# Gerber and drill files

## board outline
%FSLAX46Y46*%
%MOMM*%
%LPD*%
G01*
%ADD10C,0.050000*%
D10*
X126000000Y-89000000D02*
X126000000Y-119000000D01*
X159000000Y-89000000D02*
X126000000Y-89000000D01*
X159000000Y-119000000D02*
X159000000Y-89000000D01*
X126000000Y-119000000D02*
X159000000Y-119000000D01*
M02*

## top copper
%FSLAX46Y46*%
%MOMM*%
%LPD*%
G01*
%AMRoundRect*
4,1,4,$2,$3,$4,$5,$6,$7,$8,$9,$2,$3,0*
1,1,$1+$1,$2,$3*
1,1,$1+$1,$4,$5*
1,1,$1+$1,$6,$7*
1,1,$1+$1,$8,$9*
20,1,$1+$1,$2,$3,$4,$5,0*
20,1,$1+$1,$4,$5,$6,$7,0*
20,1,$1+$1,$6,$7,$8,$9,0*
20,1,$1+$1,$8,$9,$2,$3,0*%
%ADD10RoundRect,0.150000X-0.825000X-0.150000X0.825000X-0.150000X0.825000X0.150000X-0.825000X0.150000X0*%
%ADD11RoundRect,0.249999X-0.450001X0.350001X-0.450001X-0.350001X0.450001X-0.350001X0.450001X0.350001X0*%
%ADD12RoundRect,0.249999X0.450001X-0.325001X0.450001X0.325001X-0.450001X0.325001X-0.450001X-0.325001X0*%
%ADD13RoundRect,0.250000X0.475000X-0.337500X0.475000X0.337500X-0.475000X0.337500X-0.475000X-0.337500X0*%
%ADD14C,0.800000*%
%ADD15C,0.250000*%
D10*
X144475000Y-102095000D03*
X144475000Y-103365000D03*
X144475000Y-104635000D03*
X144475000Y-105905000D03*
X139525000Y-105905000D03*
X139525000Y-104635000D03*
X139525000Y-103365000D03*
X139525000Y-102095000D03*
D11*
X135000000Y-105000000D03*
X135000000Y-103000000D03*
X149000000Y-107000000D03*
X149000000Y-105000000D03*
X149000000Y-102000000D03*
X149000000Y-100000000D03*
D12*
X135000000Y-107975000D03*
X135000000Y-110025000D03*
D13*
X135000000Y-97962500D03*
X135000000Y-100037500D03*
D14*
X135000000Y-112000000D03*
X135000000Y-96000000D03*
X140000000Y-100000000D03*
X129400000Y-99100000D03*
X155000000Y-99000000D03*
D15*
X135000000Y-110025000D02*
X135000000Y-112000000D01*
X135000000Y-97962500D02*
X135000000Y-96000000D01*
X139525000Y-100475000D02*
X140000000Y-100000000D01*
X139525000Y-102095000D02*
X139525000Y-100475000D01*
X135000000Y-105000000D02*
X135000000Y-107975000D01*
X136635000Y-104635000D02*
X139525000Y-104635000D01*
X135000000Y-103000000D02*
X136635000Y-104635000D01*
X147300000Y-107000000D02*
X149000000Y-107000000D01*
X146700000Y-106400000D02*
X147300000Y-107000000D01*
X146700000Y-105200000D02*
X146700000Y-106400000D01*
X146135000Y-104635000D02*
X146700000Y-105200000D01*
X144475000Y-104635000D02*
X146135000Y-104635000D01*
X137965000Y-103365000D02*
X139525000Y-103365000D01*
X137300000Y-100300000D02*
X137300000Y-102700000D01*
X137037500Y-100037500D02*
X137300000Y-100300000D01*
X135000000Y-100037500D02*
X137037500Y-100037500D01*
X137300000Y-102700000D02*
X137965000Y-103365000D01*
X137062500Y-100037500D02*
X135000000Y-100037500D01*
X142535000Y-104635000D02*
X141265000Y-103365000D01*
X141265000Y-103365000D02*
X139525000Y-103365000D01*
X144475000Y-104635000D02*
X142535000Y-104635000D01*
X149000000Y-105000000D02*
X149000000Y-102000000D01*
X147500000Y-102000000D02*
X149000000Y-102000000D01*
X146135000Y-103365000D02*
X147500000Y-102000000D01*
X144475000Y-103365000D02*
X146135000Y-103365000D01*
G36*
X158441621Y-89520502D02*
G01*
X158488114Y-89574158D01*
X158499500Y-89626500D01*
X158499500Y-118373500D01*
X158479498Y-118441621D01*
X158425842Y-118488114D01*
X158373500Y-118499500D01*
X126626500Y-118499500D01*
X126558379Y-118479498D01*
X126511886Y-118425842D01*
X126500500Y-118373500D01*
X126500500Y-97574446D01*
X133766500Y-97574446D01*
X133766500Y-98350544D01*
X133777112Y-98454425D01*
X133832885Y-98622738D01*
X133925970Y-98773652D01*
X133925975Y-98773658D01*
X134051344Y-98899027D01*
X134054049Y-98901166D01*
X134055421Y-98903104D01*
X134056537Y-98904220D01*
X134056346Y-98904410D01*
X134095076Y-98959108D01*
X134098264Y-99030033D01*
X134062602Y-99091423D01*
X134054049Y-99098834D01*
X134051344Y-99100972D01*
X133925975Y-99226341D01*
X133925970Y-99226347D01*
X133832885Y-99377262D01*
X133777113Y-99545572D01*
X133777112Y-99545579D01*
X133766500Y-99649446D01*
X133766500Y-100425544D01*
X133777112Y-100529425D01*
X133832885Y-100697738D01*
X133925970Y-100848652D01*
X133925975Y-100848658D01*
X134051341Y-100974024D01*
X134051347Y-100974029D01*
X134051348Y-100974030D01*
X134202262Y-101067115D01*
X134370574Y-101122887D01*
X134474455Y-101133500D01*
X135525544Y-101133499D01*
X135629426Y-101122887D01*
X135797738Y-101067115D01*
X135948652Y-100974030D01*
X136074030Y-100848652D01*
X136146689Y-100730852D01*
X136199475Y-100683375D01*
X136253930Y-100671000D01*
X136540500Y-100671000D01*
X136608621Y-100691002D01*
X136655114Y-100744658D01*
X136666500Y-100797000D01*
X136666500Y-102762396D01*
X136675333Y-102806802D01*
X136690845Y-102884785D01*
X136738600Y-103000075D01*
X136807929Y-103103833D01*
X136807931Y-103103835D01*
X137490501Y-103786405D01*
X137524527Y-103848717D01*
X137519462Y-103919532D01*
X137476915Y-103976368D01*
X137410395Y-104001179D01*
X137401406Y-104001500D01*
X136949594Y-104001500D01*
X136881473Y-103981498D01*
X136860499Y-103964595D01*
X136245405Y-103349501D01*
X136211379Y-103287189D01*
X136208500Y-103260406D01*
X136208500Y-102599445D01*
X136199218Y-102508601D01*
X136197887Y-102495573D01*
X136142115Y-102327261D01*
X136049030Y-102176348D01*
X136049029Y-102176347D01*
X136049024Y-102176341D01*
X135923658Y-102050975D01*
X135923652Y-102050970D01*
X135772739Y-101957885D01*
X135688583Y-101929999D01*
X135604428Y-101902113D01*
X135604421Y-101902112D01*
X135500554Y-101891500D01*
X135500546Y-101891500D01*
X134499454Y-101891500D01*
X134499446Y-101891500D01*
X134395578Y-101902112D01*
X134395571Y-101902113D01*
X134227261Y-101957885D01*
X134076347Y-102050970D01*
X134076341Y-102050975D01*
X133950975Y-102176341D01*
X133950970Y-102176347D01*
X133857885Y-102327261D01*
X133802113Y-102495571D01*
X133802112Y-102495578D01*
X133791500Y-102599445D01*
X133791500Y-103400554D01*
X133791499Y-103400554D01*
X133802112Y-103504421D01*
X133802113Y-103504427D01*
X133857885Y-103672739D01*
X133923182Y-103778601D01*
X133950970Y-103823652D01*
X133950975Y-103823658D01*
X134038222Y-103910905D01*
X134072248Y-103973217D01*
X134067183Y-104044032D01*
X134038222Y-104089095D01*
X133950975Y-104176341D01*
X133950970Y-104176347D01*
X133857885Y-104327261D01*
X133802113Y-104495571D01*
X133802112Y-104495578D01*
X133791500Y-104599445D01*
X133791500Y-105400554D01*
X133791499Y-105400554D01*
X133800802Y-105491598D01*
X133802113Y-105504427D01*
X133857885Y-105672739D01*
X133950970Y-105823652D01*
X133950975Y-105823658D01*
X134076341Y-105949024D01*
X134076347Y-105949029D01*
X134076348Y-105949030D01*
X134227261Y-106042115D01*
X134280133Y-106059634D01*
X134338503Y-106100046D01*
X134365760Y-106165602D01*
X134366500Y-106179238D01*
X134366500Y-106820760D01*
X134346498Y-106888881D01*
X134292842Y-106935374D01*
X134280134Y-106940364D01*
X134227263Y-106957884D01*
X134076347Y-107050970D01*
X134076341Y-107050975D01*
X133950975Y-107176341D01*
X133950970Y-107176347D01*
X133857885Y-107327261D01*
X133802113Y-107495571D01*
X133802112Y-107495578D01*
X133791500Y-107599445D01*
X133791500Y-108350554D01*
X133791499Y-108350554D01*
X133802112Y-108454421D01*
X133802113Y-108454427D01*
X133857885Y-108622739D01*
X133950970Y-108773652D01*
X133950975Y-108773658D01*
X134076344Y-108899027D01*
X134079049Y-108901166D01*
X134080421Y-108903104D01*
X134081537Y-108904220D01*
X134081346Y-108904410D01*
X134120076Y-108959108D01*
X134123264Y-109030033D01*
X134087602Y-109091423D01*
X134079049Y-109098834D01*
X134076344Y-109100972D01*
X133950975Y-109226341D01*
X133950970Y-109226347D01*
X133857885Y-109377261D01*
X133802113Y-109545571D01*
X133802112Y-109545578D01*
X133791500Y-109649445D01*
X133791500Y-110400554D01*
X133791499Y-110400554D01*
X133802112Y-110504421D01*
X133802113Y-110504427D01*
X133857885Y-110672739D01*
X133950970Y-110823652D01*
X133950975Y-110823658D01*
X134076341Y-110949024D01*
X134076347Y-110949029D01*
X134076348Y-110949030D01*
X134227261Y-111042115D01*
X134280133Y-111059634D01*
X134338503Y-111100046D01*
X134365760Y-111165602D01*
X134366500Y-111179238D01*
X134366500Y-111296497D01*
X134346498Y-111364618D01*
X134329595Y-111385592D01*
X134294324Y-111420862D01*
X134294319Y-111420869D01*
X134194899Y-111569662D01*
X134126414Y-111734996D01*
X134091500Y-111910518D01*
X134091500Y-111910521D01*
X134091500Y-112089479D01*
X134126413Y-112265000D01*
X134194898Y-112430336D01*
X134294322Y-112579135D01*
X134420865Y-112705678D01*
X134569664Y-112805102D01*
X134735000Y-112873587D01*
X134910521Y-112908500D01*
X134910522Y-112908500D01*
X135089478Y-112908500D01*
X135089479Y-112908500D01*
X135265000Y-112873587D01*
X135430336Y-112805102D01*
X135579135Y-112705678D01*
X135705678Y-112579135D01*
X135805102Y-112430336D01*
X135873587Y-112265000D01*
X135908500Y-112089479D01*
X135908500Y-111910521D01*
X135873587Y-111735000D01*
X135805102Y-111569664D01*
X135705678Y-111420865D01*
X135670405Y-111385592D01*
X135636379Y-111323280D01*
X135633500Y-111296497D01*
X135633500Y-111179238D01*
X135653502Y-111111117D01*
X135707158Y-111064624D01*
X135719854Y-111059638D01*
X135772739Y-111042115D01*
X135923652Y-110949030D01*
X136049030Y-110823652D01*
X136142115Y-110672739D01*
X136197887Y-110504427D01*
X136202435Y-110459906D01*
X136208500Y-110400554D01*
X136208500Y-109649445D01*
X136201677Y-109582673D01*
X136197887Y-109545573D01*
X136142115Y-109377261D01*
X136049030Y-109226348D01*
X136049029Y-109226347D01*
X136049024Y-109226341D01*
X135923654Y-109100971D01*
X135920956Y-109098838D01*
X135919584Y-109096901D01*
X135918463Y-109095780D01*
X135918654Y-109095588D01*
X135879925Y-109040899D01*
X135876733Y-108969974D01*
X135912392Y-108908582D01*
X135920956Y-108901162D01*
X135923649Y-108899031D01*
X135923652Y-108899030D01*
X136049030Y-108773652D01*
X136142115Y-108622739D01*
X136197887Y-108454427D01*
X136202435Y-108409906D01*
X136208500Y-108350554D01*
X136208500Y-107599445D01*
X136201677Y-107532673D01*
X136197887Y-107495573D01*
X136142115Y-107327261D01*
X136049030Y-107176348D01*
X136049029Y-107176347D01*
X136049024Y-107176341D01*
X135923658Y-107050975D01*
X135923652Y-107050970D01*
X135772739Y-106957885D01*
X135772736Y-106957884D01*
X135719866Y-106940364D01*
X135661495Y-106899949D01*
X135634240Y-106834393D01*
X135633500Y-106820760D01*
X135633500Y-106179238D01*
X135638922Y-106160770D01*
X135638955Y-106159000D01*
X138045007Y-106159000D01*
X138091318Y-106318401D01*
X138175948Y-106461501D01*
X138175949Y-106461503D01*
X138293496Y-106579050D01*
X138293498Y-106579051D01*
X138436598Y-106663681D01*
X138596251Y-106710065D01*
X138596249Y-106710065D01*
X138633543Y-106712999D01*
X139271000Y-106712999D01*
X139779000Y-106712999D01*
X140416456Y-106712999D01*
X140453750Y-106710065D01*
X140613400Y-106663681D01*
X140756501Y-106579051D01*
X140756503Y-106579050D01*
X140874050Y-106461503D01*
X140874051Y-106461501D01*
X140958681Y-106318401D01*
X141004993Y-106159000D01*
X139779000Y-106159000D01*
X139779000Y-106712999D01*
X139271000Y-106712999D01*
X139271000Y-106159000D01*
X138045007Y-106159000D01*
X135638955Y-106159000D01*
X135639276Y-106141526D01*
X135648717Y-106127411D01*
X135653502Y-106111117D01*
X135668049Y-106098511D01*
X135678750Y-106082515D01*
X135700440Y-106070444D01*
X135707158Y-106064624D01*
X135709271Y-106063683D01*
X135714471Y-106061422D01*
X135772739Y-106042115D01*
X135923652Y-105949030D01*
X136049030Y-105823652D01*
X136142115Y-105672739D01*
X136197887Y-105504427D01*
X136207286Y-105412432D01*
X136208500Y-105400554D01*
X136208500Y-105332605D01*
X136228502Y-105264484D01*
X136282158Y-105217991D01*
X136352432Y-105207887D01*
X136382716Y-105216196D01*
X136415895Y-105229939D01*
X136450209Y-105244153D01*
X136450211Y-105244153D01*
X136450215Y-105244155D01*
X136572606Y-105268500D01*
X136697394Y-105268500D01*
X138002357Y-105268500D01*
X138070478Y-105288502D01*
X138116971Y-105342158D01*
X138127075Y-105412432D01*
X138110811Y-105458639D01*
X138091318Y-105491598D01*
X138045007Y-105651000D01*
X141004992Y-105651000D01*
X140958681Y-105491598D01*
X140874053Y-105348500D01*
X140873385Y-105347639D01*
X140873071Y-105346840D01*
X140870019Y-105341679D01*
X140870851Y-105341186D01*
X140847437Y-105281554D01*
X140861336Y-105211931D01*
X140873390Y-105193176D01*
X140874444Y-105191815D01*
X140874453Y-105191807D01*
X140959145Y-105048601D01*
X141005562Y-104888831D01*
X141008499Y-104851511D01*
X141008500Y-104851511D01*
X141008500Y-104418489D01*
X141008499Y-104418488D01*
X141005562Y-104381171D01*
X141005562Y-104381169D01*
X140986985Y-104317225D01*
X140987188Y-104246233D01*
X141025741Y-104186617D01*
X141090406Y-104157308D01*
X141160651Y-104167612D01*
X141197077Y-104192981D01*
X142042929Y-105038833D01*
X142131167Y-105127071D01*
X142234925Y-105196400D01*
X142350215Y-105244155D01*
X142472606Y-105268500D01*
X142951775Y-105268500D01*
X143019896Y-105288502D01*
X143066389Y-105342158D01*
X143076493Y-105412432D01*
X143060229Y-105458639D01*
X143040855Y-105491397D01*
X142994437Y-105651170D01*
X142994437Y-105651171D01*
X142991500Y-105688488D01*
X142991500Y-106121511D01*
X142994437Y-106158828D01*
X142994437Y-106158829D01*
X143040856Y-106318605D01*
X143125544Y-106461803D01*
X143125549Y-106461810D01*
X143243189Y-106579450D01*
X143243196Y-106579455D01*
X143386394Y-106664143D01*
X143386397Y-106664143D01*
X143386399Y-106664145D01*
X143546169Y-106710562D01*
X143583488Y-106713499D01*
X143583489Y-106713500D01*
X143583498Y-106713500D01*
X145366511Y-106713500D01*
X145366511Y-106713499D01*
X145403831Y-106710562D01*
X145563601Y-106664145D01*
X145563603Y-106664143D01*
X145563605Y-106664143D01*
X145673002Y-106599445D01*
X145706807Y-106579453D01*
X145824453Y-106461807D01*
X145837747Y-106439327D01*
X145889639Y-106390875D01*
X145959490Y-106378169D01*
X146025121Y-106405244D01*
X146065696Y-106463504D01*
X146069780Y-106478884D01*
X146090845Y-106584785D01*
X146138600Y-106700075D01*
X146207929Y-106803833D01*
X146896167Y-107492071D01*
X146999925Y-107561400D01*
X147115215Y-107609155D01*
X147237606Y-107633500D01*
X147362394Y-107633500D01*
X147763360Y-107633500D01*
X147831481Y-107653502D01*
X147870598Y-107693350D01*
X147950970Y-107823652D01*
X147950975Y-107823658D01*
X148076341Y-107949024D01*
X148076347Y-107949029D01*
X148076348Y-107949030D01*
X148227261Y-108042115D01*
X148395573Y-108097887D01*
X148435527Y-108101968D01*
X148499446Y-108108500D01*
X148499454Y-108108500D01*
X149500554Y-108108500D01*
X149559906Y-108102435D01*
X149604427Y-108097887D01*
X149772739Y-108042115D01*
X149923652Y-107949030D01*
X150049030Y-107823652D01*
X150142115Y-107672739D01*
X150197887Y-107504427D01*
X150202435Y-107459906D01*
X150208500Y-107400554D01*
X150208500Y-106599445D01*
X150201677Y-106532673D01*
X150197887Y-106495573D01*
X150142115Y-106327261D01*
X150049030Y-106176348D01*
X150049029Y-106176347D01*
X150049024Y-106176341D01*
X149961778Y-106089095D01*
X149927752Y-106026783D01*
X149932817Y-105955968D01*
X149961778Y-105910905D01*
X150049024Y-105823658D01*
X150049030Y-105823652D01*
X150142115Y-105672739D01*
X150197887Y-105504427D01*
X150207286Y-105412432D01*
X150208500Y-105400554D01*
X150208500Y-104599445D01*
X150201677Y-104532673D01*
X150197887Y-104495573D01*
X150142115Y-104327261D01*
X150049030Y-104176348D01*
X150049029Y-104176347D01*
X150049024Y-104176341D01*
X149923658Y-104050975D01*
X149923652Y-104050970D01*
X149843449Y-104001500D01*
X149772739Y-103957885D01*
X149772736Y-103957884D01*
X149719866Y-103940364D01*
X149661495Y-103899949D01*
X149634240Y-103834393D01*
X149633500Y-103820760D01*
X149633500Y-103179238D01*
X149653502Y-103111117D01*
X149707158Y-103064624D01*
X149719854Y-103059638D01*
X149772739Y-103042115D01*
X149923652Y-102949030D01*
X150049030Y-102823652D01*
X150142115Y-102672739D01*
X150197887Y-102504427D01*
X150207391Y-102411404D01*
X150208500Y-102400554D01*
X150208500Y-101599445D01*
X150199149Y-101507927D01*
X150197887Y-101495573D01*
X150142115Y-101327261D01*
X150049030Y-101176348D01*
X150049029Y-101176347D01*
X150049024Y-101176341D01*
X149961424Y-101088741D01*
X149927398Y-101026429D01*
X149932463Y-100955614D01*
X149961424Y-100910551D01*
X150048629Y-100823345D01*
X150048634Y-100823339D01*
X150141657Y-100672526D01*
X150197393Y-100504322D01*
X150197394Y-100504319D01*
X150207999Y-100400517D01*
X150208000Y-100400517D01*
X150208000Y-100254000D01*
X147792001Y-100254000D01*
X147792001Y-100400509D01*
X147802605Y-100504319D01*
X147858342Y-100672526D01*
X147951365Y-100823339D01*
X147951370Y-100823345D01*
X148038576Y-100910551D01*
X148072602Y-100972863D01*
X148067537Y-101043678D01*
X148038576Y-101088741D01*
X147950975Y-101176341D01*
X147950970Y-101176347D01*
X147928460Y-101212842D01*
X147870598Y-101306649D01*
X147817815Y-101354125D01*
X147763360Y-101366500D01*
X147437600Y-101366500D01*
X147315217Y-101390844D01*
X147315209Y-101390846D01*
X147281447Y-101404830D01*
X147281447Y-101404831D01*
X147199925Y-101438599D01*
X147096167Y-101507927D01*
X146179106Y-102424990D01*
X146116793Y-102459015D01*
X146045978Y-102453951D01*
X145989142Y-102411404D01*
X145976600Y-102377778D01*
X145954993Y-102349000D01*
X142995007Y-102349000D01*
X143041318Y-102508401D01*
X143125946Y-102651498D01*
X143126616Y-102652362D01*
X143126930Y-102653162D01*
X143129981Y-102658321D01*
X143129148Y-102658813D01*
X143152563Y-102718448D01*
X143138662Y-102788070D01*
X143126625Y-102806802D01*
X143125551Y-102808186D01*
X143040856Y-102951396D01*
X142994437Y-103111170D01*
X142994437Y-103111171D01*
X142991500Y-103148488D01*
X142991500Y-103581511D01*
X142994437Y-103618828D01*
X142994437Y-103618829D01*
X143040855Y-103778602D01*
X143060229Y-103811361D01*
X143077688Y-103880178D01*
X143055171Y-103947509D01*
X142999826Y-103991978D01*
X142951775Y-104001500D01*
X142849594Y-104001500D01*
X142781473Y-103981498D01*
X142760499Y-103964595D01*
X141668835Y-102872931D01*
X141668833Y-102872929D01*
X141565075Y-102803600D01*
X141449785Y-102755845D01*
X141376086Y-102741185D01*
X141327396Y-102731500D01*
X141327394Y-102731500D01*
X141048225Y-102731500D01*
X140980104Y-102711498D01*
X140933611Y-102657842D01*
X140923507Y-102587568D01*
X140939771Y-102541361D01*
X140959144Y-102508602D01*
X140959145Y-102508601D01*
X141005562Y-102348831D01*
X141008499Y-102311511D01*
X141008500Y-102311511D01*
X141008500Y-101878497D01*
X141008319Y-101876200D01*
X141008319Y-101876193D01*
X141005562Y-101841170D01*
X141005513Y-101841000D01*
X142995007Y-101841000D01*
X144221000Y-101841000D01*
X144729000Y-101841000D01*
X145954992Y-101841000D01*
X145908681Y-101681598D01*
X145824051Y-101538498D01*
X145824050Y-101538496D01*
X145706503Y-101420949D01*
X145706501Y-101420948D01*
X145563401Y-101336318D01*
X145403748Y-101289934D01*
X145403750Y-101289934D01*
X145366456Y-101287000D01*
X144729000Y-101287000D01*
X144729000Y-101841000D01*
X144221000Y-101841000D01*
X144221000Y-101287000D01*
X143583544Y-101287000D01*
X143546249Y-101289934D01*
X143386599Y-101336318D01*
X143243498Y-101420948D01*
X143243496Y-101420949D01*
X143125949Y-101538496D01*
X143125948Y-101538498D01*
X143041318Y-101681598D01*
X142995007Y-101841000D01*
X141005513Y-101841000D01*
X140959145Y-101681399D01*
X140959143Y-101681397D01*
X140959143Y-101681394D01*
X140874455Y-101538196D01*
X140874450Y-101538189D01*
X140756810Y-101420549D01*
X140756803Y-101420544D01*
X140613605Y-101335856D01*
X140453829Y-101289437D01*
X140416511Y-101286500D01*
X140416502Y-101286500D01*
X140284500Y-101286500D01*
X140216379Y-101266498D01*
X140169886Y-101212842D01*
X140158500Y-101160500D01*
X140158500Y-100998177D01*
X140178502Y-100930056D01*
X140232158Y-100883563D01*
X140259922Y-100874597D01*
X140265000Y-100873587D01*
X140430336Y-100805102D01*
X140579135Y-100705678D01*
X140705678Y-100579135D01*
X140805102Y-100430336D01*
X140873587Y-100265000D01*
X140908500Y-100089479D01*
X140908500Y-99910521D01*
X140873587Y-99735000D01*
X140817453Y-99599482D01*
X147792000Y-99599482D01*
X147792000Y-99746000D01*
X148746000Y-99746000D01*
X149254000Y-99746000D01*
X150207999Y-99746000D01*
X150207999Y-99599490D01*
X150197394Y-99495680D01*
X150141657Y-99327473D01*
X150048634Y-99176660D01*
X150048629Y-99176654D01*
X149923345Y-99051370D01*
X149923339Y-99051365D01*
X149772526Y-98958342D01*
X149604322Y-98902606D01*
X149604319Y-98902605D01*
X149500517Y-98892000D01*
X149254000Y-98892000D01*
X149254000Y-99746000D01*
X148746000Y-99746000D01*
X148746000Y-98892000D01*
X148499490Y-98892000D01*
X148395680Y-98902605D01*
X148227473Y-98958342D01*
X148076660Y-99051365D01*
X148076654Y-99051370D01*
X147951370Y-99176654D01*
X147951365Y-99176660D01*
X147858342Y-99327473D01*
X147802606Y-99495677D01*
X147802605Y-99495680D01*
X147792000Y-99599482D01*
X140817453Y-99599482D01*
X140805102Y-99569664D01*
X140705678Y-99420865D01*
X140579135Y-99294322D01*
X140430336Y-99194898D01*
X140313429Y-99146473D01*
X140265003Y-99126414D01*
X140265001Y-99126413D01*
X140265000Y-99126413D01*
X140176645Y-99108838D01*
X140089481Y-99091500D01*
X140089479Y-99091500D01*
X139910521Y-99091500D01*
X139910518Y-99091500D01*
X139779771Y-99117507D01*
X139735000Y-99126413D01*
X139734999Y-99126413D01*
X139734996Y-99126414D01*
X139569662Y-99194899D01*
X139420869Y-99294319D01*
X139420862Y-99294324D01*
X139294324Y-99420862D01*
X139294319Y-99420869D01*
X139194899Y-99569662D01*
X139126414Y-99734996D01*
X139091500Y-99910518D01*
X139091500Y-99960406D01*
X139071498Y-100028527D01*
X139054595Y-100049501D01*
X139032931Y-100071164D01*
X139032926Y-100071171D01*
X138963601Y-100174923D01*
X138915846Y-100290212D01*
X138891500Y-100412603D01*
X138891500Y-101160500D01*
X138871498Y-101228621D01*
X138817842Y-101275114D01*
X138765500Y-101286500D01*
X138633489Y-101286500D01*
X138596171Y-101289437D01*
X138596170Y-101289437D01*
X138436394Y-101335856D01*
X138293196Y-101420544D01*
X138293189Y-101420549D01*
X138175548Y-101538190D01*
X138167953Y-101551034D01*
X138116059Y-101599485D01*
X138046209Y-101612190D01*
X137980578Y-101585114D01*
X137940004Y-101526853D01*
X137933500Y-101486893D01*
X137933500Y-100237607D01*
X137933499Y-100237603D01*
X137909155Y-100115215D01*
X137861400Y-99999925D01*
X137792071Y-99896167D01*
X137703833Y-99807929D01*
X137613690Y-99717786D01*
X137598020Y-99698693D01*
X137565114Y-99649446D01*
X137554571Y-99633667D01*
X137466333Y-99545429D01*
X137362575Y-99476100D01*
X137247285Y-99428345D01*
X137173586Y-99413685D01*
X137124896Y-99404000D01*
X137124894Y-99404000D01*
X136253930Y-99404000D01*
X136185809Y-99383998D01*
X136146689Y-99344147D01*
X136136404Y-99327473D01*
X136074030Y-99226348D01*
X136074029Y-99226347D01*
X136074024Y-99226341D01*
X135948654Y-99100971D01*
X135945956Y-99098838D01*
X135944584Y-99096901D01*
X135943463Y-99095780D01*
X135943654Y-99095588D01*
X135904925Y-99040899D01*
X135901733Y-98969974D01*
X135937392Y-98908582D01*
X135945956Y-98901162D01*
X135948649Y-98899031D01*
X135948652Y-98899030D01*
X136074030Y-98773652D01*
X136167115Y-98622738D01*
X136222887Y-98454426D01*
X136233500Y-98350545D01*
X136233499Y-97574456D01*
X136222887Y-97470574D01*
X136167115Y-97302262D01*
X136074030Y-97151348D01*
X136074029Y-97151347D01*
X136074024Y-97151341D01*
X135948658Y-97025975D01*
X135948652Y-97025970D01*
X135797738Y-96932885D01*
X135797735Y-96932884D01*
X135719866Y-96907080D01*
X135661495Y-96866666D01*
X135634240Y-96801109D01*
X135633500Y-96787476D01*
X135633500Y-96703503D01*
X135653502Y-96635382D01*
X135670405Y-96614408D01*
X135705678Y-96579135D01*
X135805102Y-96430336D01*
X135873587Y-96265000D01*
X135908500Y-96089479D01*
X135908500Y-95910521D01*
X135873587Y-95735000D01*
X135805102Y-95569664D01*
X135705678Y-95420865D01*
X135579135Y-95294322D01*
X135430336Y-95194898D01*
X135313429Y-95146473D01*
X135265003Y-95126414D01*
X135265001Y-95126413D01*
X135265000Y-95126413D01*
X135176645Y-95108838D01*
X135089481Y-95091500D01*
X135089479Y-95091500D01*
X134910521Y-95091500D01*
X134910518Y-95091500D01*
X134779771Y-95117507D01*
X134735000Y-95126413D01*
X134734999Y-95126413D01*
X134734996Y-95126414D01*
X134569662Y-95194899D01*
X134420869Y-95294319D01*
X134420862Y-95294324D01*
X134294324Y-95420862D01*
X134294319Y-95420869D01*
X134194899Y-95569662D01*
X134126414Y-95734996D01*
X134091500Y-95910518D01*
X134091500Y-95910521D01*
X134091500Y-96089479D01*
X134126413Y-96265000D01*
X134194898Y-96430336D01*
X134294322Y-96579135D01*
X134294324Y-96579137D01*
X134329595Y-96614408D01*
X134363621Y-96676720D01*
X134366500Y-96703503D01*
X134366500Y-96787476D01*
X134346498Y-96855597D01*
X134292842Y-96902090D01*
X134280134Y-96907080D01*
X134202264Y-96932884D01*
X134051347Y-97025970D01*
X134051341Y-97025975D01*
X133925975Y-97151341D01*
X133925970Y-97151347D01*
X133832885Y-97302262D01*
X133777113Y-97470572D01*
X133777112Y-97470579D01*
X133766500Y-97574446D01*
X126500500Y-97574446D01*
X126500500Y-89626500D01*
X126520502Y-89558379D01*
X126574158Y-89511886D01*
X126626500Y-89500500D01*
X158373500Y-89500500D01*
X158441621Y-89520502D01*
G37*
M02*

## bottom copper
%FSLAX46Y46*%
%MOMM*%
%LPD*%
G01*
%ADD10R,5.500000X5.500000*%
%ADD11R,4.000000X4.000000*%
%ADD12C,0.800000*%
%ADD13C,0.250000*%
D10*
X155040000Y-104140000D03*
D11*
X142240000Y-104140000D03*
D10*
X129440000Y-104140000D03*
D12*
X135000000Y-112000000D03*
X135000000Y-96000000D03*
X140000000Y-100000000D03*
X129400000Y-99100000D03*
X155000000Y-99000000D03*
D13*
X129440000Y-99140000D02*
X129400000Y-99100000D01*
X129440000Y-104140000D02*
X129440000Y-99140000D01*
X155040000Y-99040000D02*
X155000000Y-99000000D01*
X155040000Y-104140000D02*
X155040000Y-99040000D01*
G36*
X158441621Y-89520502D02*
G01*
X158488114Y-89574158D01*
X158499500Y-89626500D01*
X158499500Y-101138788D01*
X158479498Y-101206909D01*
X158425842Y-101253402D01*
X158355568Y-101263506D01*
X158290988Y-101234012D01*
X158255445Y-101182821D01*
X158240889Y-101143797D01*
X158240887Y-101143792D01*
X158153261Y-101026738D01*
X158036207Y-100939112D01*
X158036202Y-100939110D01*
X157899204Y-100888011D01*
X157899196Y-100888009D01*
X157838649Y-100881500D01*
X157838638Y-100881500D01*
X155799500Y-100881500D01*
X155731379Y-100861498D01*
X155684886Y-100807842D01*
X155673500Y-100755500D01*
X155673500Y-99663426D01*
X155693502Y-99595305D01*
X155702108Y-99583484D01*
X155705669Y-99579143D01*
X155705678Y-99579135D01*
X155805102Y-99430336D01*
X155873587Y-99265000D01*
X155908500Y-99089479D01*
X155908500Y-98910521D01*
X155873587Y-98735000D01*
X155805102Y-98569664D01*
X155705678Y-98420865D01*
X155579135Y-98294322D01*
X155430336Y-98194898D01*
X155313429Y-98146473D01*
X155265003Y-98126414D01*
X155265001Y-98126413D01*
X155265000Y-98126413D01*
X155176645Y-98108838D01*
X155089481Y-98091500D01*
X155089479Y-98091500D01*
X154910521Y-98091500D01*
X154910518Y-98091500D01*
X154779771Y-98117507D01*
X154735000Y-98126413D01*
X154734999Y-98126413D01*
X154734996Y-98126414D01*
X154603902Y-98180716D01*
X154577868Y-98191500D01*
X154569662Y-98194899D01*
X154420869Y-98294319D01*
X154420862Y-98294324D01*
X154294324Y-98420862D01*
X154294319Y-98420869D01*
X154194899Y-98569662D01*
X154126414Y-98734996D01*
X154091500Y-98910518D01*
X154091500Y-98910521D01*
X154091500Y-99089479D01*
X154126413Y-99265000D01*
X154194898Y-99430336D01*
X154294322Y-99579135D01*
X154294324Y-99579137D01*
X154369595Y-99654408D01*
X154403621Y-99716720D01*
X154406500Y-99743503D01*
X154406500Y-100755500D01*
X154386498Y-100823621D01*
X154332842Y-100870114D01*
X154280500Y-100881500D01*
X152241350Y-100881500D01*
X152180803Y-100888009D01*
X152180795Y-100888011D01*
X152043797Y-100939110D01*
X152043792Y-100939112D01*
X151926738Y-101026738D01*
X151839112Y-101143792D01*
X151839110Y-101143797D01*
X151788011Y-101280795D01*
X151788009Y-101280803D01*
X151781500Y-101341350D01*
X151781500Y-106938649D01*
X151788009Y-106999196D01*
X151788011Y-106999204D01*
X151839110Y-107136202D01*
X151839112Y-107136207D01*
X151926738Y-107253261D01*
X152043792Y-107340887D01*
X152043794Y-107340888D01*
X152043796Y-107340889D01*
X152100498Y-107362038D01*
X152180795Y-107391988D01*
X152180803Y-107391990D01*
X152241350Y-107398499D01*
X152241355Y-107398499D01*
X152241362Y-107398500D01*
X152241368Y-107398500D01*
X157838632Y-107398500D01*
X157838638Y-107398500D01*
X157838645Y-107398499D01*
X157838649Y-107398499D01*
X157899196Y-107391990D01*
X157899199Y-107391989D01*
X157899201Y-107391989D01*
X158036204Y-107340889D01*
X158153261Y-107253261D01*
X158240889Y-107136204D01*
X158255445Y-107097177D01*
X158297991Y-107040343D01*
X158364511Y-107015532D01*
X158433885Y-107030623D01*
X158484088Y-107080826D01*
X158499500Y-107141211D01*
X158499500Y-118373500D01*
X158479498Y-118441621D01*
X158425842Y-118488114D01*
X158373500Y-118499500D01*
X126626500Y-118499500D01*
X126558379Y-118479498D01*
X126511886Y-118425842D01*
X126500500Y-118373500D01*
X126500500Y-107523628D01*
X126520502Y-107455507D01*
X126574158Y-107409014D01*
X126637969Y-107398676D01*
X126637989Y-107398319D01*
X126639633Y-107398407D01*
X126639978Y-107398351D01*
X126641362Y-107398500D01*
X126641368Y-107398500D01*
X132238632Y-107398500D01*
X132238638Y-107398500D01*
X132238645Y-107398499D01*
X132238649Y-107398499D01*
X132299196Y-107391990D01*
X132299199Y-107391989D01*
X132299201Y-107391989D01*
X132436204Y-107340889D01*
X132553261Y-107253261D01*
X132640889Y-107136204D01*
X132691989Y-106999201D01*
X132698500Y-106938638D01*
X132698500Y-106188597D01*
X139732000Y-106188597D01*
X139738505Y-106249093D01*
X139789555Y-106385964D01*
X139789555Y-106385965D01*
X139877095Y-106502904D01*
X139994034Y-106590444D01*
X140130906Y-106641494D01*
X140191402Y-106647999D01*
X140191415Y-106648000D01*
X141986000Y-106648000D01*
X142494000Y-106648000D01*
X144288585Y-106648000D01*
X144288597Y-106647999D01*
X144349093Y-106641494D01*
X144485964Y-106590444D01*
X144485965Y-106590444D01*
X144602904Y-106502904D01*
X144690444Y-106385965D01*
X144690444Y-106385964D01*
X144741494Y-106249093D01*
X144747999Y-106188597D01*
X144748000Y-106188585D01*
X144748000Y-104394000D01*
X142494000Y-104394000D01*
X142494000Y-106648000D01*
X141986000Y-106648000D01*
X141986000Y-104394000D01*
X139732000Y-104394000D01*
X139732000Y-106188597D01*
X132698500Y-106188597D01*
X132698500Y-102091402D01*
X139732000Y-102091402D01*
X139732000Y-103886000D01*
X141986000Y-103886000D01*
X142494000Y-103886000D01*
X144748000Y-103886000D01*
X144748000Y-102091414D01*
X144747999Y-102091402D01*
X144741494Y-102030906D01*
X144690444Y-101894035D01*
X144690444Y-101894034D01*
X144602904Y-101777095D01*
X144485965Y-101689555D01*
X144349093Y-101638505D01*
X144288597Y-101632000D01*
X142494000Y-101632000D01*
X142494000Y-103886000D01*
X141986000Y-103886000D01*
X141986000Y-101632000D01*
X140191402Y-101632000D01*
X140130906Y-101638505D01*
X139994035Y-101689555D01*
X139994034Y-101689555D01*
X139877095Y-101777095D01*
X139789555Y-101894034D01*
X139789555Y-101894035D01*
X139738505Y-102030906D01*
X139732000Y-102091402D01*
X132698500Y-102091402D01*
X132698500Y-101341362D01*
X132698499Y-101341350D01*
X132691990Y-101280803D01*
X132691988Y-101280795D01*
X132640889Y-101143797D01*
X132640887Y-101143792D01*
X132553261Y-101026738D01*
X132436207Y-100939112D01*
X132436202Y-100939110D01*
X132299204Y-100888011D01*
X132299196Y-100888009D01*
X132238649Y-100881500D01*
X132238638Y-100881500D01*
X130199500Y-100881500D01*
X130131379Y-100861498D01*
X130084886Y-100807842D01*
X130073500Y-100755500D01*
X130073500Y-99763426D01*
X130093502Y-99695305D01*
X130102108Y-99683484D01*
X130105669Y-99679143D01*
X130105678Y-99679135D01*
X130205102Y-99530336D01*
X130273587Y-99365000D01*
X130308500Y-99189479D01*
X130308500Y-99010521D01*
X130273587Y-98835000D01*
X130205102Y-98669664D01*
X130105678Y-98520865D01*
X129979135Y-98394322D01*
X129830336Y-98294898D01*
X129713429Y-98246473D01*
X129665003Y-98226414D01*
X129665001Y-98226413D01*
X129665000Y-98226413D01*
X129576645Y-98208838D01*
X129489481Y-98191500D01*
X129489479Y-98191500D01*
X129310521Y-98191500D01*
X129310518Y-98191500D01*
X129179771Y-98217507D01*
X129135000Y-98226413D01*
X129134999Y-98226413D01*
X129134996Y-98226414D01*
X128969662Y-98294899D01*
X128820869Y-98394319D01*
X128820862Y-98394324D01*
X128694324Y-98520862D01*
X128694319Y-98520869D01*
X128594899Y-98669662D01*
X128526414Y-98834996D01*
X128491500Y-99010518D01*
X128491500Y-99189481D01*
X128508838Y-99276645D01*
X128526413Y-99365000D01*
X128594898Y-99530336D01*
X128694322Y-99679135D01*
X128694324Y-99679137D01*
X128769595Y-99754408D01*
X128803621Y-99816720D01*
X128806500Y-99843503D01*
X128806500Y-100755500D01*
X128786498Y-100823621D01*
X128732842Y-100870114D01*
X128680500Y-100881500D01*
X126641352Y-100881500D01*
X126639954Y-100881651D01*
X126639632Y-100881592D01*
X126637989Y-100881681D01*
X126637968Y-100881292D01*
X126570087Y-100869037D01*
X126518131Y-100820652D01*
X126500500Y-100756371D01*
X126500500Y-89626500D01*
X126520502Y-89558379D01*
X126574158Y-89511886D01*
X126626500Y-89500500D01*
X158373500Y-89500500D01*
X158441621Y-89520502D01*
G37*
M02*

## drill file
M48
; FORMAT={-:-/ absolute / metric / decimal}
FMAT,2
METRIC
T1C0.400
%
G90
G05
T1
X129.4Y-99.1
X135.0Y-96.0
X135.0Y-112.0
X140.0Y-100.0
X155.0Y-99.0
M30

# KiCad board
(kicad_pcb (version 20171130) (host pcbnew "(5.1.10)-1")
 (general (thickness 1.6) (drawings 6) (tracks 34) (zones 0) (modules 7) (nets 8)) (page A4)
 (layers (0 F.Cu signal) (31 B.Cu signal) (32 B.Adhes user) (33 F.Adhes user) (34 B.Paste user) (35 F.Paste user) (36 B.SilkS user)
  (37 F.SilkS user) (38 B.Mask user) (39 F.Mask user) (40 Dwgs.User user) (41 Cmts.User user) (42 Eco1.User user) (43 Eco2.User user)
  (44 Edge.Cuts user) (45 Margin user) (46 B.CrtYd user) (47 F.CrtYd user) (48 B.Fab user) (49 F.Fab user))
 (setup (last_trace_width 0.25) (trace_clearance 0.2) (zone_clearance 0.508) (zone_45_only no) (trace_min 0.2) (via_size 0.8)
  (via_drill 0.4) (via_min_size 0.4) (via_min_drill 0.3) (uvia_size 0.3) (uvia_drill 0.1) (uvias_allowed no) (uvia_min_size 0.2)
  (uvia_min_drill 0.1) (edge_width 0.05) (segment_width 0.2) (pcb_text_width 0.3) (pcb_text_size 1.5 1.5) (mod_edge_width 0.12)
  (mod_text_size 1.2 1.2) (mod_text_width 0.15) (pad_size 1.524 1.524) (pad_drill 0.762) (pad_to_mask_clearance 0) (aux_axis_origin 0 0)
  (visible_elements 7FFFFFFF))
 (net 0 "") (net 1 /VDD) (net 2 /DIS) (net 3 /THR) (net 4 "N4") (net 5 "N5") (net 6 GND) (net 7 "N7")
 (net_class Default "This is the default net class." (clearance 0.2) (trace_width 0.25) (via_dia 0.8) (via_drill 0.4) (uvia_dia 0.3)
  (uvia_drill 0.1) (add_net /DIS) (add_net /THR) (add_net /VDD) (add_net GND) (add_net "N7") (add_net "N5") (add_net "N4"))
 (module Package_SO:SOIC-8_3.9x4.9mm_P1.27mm (layer F.Cu) (at 142 104)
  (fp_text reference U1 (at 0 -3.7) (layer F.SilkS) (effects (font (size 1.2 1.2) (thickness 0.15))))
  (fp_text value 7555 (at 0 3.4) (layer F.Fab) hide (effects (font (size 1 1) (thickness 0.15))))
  (pad 8 smd roundrect (at 2.475 -1.905) (size 1.95 0.6) (layers F.Cu F.Paste F.Mask) (roundrect_rratio 0.25) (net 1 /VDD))
  (pad 7 smd roundrect (at 2.475 -0.635) (size 1.95 0.6) (layers F.Cu F.Paste F.Mask) (roundrect_rratio 0.25) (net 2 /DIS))
  (pad 6 smd roundrect (at 2.475 0.635) (size 1.95 0.6) (layers F.Cu F.Paste F.Mask) (roundrect_rratio 0.25) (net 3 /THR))
  (pad 5 smd roundrect (at 2.475 1.905) (size 1.95 0.6) (layers F.Cu F.Paste F.Mask) (roundrect_rratio 0.25) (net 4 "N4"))
  (pad 4 smd roundrect (at -2.475 1.905) (size 1.95 0.6) (layers F.Cu F.Paste F.Mask) (roundrect_rratio 0.25) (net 1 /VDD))
  (pad 3 smd roundrect (at -2.475 0.635) (size 1.95 0.6) (layers F.Cu F.Paste F.Mask) (roundrect_rratio 0.25) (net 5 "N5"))
  (pad 2 smd roundrect (at -2.475 -0.635) (size 1.95 0.6) (layers F.Cu F.Paste F.Mask) (roundrect_rratio 0.25) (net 3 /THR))
  (pad 1 smd roundrect (at -2.475 -1.905) (size 1.95 0.6) (layers F.Cu F.Paste F.Mask) (roundrect_rratio 0.25) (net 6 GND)))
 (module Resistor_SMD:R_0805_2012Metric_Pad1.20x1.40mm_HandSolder (layer F.Cu) (at 135 104 270)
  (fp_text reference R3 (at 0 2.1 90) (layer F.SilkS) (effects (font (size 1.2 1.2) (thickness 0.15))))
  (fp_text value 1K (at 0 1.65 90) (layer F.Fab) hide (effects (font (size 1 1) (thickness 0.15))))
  (pad 2 smd roundrect (at 1 0 270) (size 1.2 1.4) (layers F.Cu F.Paste F.Mask) (roundrect_rratio 0.2083325) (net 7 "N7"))
  (pad 1 smd roundrect (at -1 0 270) (size 1.2 1.4) (layers F.Cu F.Paste F.Mask) (roundrect_rratio 0.2083325) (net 5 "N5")))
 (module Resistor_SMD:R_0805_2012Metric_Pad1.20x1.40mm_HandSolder (layer F.Cu) (at 149 106 270)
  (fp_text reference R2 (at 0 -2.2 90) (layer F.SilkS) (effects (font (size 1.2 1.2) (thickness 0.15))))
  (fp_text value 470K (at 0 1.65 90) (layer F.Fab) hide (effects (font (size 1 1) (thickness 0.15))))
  (pad 2 smd roundrect (at 1 0 270) (size 1.2 1.4) (layers F.Cu F.Paste F.Mask) (roundrect_rratio 0.2083325) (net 3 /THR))
  (pad 1 smd roundrect (at -1 0 270) (size 1.2 1.4) (layers F.Cu F.Paste F.Mask) (roundrect_rratio 0.2083325) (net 2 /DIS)))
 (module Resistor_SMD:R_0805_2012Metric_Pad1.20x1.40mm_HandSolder (layer F.Cu) (at 149 101 270)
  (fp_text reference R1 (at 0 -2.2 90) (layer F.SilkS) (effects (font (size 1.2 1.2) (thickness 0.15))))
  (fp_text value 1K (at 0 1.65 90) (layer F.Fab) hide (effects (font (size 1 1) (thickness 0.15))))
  (pad 2 smd roundrect (at 1 0 270) (size 1.2 1.4) (layers F.Cu F.Paste F.Mask) (roundrect_rratio 0.2083325) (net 2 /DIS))
  (pad 1 smd roundrect (at -1 0 270) (size 1.2 1.4) (layers F.Cu F.Paste F.Mask) (roundrect_rratio 0.2083325) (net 1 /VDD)))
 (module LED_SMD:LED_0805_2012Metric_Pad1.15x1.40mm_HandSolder (layer F.Cu) (at 135 109 90)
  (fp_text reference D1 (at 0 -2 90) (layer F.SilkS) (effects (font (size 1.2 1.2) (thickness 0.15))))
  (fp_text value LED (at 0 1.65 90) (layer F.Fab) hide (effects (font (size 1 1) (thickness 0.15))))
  (pad 2 smd roundrect (at 1.025 0 90) (size 1.15 1.4) (layers F.Cu F.Paste F.Mask) (roundrect_rratio 0.2173904347826087) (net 7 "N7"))
  (pad 1 smd roundrect (at -1.025 0 90) (size 1.15 1.4) (layers F.Cu F.Paste F.Mask) (roundrect_rratio 0.2173904347826087) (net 6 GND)))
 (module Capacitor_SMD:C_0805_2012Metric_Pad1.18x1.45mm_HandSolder (layer F.Cu) (at 135 99 90)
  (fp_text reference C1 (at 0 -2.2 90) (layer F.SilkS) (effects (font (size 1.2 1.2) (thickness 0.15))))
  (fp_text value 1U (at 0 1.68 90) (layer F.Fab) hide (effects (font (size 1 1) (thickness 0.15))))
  (pad 2 smd roundrect (at 1.0375 0 90) (size 1.175 1.45) (layers F.Cu F.Paste F.Mask) (roundrect_rratio 0.2127659574468085) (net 6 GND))
  (pad 1 smd roundrect (at -1.0375 0 90) (size 1.175 1.45) (layers F.Cu F.Paste F.Mask) (roundrect_rratio 0.2127659574468085) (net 3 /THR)))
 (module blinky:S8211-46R (layer B.Cu) (at 142.24 104.14)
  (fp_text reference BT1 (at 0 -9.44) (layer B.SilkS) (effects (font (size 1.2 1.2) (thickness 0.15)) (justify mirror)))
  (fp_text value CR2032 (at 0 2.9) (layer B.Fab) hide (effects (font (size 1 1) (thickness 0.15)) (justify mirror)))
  (pad 1 smd rect (at 12.8 0) (size 5.5 5.5) (layers B.Cu B.Paste B.Mask) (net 1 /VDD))
  (pad 2 smd rect (at 0 0 270) (size 4 4) (layers B.Cu B.Paste B.Mask) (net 6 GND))
  (pad 1 smd rect (at -12.8 0) (size 5.5 5.5) (layers B.Cu B.Paste B.Mask) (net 1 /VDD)))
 (gr_line (start 126 89) (end 126 119) (layer Edge.Cuts) (width 0.05))
 (gr_line (start 159 89) (end 126 89) (layer Edge.Cuts) (width 0.05))
 (gr_line (start 159 119) (end 159 89) (layer Edge.Cuts) (width 0.05))
 (gr_line (start 126 119) (end 159 119) (layer Edge.Cuts) (width 0.05))
 (via (at 135 112) (size 0.8) (drill 0.4) (layers F.Cu B.Cu) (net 6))
 (segment (start 135 110.025) (end 135 112) (width 0.25) (layer F.Cu) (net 6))
 (via (at 135 96) (size 0.8) (drill 0.4) (layers F.Cu B.Cu) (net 6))
 (segment (start 135 97.9625) (end 135 96) (width 0.25) (layer F.Cu) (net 6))
 (via (at 140 100) (size 0.8) (drill 0.4) (layers F.Cu B.Cu) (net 6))
 (segment (start 139.525 100.475) (end 140 100) (width 0.25) (layer F.Cu) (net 6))
 (segment (start 139.525 102.095) (end 139.525 100.475) (width 0.25) (layer F.Cu) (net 6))
 (segment (start 135 105) (end 135 107.975) (width 0.25) (layer F.Cu) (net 7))
 (segment (start 136.635 104.635) (end 139.525 104.635) (width 0.25) (layer F.Cu) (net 5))
 (segment (start 135 103) (end 136.635 104.635) (width 0.25) (layer F.Cu) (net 5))
 (via (at 129.4 99.1) (size 0.8) (drill 0.4) (layers F.Cu B.Cu) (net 1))
 (segment (start 129.44 99.14) (end 129.4 99.1) (width 0.25) (layer B.Cu) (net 1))
 (segment (start 129.44 104.14) (end 129.44 99.14) (width 0.25) (layer B.Cu) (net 1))
 (segment (start 155.04 99.04) (end 155 99) (width 0.25) (layer B.Cu) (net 1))
 (via (at 155 99) (size 0.8) (drill 0.4) (layers F.Cu B.Cu) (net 1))
 (segment (start 155.04 104.14) (end 155.04 99.04) (width 0.25) (layer B.Cu) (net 1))
 (segment (start 147.3 107) (end 149 107) (width 0.25) (layer F.Cu) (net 3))
 (segment (start 146.7 106.4) (end 147.3 107) (width 0.25) (layer F.Cu) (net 3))
 (segment (start 146.7 105.2) (end 146.7 106.4) (width 0.25) (layer F.Cu) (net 3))
 (segment (start 146.135 104.635) (end 146.7 105.2) (width 0.25) (layer F.Cu) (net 3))
 (segment (start 144.475 104.635) (end 146.135 104.635) (width 0.25) (layer F.Cu) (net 3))
 (segment (start 137.965 103.365) (end 139.525 103.365) (width 0.25) (layer F.Cu) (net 3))
 (segment (start 137.3 100.3) (end 137.3 102.7) (width 0.25) (layer F.Cu) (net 3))
 (segment (start 137.0375 100.0375) (end 137.3 100.3) (width 0.25) (layer F.Cu) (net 3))
 (segment (start 135 100.0375) (end 137.0375 100.0375) (width 0.25) (layer F.Cu) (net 3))
 (segment (start 137.3 102.7) (end 137.965 103.365) (width 0.25) (layer F.Cu) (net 3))
 (segment (start 137.0625 100.0375) (end 135 100.0375) (width 0.25) (layer F.Cu) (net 3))
 (segment (start 142.535 104.635) (end 141.265 103.365) (width 0.25) (layer F.Cu) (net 3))
 (segment (start 141.265 103.365) (end 139.525 103.365) (width 0.25) (layer F.Cu) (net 3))
 (segment (start 144.475 104.635) (end 142.535 104.635) (width 0.25) (layer F.Cu) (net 3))
 (segment (start 149 105) (end 149 102) (width 0.25) (layer F.Cu) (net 2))
 (segment (start 147.5 102) (end 149 102) (width 0.25) (layer F.Cu) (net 2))
 (segment (start 146.135 103.365) (end 147.5 102) (width 0.25) (layer F.Cu) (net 2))
 (segment (start 144.475 103.365) (end 146.135 103.365) (width 0.25) (layer F.Cu) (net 2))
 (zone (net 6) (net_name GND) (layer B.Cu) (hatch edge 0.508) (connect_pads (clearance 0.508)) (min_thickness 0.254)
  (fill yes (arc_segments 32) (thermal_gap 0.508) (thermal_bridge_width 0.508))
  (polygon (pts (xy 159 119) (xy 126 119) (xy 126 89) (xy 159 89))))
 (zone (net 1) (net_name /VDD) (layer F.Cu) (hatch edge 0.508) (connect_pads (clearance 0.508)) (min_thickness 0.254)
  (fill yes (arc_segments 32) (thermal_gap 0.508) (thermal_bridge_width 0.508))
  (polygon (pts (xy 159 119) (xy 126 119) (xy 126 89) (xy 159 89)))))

